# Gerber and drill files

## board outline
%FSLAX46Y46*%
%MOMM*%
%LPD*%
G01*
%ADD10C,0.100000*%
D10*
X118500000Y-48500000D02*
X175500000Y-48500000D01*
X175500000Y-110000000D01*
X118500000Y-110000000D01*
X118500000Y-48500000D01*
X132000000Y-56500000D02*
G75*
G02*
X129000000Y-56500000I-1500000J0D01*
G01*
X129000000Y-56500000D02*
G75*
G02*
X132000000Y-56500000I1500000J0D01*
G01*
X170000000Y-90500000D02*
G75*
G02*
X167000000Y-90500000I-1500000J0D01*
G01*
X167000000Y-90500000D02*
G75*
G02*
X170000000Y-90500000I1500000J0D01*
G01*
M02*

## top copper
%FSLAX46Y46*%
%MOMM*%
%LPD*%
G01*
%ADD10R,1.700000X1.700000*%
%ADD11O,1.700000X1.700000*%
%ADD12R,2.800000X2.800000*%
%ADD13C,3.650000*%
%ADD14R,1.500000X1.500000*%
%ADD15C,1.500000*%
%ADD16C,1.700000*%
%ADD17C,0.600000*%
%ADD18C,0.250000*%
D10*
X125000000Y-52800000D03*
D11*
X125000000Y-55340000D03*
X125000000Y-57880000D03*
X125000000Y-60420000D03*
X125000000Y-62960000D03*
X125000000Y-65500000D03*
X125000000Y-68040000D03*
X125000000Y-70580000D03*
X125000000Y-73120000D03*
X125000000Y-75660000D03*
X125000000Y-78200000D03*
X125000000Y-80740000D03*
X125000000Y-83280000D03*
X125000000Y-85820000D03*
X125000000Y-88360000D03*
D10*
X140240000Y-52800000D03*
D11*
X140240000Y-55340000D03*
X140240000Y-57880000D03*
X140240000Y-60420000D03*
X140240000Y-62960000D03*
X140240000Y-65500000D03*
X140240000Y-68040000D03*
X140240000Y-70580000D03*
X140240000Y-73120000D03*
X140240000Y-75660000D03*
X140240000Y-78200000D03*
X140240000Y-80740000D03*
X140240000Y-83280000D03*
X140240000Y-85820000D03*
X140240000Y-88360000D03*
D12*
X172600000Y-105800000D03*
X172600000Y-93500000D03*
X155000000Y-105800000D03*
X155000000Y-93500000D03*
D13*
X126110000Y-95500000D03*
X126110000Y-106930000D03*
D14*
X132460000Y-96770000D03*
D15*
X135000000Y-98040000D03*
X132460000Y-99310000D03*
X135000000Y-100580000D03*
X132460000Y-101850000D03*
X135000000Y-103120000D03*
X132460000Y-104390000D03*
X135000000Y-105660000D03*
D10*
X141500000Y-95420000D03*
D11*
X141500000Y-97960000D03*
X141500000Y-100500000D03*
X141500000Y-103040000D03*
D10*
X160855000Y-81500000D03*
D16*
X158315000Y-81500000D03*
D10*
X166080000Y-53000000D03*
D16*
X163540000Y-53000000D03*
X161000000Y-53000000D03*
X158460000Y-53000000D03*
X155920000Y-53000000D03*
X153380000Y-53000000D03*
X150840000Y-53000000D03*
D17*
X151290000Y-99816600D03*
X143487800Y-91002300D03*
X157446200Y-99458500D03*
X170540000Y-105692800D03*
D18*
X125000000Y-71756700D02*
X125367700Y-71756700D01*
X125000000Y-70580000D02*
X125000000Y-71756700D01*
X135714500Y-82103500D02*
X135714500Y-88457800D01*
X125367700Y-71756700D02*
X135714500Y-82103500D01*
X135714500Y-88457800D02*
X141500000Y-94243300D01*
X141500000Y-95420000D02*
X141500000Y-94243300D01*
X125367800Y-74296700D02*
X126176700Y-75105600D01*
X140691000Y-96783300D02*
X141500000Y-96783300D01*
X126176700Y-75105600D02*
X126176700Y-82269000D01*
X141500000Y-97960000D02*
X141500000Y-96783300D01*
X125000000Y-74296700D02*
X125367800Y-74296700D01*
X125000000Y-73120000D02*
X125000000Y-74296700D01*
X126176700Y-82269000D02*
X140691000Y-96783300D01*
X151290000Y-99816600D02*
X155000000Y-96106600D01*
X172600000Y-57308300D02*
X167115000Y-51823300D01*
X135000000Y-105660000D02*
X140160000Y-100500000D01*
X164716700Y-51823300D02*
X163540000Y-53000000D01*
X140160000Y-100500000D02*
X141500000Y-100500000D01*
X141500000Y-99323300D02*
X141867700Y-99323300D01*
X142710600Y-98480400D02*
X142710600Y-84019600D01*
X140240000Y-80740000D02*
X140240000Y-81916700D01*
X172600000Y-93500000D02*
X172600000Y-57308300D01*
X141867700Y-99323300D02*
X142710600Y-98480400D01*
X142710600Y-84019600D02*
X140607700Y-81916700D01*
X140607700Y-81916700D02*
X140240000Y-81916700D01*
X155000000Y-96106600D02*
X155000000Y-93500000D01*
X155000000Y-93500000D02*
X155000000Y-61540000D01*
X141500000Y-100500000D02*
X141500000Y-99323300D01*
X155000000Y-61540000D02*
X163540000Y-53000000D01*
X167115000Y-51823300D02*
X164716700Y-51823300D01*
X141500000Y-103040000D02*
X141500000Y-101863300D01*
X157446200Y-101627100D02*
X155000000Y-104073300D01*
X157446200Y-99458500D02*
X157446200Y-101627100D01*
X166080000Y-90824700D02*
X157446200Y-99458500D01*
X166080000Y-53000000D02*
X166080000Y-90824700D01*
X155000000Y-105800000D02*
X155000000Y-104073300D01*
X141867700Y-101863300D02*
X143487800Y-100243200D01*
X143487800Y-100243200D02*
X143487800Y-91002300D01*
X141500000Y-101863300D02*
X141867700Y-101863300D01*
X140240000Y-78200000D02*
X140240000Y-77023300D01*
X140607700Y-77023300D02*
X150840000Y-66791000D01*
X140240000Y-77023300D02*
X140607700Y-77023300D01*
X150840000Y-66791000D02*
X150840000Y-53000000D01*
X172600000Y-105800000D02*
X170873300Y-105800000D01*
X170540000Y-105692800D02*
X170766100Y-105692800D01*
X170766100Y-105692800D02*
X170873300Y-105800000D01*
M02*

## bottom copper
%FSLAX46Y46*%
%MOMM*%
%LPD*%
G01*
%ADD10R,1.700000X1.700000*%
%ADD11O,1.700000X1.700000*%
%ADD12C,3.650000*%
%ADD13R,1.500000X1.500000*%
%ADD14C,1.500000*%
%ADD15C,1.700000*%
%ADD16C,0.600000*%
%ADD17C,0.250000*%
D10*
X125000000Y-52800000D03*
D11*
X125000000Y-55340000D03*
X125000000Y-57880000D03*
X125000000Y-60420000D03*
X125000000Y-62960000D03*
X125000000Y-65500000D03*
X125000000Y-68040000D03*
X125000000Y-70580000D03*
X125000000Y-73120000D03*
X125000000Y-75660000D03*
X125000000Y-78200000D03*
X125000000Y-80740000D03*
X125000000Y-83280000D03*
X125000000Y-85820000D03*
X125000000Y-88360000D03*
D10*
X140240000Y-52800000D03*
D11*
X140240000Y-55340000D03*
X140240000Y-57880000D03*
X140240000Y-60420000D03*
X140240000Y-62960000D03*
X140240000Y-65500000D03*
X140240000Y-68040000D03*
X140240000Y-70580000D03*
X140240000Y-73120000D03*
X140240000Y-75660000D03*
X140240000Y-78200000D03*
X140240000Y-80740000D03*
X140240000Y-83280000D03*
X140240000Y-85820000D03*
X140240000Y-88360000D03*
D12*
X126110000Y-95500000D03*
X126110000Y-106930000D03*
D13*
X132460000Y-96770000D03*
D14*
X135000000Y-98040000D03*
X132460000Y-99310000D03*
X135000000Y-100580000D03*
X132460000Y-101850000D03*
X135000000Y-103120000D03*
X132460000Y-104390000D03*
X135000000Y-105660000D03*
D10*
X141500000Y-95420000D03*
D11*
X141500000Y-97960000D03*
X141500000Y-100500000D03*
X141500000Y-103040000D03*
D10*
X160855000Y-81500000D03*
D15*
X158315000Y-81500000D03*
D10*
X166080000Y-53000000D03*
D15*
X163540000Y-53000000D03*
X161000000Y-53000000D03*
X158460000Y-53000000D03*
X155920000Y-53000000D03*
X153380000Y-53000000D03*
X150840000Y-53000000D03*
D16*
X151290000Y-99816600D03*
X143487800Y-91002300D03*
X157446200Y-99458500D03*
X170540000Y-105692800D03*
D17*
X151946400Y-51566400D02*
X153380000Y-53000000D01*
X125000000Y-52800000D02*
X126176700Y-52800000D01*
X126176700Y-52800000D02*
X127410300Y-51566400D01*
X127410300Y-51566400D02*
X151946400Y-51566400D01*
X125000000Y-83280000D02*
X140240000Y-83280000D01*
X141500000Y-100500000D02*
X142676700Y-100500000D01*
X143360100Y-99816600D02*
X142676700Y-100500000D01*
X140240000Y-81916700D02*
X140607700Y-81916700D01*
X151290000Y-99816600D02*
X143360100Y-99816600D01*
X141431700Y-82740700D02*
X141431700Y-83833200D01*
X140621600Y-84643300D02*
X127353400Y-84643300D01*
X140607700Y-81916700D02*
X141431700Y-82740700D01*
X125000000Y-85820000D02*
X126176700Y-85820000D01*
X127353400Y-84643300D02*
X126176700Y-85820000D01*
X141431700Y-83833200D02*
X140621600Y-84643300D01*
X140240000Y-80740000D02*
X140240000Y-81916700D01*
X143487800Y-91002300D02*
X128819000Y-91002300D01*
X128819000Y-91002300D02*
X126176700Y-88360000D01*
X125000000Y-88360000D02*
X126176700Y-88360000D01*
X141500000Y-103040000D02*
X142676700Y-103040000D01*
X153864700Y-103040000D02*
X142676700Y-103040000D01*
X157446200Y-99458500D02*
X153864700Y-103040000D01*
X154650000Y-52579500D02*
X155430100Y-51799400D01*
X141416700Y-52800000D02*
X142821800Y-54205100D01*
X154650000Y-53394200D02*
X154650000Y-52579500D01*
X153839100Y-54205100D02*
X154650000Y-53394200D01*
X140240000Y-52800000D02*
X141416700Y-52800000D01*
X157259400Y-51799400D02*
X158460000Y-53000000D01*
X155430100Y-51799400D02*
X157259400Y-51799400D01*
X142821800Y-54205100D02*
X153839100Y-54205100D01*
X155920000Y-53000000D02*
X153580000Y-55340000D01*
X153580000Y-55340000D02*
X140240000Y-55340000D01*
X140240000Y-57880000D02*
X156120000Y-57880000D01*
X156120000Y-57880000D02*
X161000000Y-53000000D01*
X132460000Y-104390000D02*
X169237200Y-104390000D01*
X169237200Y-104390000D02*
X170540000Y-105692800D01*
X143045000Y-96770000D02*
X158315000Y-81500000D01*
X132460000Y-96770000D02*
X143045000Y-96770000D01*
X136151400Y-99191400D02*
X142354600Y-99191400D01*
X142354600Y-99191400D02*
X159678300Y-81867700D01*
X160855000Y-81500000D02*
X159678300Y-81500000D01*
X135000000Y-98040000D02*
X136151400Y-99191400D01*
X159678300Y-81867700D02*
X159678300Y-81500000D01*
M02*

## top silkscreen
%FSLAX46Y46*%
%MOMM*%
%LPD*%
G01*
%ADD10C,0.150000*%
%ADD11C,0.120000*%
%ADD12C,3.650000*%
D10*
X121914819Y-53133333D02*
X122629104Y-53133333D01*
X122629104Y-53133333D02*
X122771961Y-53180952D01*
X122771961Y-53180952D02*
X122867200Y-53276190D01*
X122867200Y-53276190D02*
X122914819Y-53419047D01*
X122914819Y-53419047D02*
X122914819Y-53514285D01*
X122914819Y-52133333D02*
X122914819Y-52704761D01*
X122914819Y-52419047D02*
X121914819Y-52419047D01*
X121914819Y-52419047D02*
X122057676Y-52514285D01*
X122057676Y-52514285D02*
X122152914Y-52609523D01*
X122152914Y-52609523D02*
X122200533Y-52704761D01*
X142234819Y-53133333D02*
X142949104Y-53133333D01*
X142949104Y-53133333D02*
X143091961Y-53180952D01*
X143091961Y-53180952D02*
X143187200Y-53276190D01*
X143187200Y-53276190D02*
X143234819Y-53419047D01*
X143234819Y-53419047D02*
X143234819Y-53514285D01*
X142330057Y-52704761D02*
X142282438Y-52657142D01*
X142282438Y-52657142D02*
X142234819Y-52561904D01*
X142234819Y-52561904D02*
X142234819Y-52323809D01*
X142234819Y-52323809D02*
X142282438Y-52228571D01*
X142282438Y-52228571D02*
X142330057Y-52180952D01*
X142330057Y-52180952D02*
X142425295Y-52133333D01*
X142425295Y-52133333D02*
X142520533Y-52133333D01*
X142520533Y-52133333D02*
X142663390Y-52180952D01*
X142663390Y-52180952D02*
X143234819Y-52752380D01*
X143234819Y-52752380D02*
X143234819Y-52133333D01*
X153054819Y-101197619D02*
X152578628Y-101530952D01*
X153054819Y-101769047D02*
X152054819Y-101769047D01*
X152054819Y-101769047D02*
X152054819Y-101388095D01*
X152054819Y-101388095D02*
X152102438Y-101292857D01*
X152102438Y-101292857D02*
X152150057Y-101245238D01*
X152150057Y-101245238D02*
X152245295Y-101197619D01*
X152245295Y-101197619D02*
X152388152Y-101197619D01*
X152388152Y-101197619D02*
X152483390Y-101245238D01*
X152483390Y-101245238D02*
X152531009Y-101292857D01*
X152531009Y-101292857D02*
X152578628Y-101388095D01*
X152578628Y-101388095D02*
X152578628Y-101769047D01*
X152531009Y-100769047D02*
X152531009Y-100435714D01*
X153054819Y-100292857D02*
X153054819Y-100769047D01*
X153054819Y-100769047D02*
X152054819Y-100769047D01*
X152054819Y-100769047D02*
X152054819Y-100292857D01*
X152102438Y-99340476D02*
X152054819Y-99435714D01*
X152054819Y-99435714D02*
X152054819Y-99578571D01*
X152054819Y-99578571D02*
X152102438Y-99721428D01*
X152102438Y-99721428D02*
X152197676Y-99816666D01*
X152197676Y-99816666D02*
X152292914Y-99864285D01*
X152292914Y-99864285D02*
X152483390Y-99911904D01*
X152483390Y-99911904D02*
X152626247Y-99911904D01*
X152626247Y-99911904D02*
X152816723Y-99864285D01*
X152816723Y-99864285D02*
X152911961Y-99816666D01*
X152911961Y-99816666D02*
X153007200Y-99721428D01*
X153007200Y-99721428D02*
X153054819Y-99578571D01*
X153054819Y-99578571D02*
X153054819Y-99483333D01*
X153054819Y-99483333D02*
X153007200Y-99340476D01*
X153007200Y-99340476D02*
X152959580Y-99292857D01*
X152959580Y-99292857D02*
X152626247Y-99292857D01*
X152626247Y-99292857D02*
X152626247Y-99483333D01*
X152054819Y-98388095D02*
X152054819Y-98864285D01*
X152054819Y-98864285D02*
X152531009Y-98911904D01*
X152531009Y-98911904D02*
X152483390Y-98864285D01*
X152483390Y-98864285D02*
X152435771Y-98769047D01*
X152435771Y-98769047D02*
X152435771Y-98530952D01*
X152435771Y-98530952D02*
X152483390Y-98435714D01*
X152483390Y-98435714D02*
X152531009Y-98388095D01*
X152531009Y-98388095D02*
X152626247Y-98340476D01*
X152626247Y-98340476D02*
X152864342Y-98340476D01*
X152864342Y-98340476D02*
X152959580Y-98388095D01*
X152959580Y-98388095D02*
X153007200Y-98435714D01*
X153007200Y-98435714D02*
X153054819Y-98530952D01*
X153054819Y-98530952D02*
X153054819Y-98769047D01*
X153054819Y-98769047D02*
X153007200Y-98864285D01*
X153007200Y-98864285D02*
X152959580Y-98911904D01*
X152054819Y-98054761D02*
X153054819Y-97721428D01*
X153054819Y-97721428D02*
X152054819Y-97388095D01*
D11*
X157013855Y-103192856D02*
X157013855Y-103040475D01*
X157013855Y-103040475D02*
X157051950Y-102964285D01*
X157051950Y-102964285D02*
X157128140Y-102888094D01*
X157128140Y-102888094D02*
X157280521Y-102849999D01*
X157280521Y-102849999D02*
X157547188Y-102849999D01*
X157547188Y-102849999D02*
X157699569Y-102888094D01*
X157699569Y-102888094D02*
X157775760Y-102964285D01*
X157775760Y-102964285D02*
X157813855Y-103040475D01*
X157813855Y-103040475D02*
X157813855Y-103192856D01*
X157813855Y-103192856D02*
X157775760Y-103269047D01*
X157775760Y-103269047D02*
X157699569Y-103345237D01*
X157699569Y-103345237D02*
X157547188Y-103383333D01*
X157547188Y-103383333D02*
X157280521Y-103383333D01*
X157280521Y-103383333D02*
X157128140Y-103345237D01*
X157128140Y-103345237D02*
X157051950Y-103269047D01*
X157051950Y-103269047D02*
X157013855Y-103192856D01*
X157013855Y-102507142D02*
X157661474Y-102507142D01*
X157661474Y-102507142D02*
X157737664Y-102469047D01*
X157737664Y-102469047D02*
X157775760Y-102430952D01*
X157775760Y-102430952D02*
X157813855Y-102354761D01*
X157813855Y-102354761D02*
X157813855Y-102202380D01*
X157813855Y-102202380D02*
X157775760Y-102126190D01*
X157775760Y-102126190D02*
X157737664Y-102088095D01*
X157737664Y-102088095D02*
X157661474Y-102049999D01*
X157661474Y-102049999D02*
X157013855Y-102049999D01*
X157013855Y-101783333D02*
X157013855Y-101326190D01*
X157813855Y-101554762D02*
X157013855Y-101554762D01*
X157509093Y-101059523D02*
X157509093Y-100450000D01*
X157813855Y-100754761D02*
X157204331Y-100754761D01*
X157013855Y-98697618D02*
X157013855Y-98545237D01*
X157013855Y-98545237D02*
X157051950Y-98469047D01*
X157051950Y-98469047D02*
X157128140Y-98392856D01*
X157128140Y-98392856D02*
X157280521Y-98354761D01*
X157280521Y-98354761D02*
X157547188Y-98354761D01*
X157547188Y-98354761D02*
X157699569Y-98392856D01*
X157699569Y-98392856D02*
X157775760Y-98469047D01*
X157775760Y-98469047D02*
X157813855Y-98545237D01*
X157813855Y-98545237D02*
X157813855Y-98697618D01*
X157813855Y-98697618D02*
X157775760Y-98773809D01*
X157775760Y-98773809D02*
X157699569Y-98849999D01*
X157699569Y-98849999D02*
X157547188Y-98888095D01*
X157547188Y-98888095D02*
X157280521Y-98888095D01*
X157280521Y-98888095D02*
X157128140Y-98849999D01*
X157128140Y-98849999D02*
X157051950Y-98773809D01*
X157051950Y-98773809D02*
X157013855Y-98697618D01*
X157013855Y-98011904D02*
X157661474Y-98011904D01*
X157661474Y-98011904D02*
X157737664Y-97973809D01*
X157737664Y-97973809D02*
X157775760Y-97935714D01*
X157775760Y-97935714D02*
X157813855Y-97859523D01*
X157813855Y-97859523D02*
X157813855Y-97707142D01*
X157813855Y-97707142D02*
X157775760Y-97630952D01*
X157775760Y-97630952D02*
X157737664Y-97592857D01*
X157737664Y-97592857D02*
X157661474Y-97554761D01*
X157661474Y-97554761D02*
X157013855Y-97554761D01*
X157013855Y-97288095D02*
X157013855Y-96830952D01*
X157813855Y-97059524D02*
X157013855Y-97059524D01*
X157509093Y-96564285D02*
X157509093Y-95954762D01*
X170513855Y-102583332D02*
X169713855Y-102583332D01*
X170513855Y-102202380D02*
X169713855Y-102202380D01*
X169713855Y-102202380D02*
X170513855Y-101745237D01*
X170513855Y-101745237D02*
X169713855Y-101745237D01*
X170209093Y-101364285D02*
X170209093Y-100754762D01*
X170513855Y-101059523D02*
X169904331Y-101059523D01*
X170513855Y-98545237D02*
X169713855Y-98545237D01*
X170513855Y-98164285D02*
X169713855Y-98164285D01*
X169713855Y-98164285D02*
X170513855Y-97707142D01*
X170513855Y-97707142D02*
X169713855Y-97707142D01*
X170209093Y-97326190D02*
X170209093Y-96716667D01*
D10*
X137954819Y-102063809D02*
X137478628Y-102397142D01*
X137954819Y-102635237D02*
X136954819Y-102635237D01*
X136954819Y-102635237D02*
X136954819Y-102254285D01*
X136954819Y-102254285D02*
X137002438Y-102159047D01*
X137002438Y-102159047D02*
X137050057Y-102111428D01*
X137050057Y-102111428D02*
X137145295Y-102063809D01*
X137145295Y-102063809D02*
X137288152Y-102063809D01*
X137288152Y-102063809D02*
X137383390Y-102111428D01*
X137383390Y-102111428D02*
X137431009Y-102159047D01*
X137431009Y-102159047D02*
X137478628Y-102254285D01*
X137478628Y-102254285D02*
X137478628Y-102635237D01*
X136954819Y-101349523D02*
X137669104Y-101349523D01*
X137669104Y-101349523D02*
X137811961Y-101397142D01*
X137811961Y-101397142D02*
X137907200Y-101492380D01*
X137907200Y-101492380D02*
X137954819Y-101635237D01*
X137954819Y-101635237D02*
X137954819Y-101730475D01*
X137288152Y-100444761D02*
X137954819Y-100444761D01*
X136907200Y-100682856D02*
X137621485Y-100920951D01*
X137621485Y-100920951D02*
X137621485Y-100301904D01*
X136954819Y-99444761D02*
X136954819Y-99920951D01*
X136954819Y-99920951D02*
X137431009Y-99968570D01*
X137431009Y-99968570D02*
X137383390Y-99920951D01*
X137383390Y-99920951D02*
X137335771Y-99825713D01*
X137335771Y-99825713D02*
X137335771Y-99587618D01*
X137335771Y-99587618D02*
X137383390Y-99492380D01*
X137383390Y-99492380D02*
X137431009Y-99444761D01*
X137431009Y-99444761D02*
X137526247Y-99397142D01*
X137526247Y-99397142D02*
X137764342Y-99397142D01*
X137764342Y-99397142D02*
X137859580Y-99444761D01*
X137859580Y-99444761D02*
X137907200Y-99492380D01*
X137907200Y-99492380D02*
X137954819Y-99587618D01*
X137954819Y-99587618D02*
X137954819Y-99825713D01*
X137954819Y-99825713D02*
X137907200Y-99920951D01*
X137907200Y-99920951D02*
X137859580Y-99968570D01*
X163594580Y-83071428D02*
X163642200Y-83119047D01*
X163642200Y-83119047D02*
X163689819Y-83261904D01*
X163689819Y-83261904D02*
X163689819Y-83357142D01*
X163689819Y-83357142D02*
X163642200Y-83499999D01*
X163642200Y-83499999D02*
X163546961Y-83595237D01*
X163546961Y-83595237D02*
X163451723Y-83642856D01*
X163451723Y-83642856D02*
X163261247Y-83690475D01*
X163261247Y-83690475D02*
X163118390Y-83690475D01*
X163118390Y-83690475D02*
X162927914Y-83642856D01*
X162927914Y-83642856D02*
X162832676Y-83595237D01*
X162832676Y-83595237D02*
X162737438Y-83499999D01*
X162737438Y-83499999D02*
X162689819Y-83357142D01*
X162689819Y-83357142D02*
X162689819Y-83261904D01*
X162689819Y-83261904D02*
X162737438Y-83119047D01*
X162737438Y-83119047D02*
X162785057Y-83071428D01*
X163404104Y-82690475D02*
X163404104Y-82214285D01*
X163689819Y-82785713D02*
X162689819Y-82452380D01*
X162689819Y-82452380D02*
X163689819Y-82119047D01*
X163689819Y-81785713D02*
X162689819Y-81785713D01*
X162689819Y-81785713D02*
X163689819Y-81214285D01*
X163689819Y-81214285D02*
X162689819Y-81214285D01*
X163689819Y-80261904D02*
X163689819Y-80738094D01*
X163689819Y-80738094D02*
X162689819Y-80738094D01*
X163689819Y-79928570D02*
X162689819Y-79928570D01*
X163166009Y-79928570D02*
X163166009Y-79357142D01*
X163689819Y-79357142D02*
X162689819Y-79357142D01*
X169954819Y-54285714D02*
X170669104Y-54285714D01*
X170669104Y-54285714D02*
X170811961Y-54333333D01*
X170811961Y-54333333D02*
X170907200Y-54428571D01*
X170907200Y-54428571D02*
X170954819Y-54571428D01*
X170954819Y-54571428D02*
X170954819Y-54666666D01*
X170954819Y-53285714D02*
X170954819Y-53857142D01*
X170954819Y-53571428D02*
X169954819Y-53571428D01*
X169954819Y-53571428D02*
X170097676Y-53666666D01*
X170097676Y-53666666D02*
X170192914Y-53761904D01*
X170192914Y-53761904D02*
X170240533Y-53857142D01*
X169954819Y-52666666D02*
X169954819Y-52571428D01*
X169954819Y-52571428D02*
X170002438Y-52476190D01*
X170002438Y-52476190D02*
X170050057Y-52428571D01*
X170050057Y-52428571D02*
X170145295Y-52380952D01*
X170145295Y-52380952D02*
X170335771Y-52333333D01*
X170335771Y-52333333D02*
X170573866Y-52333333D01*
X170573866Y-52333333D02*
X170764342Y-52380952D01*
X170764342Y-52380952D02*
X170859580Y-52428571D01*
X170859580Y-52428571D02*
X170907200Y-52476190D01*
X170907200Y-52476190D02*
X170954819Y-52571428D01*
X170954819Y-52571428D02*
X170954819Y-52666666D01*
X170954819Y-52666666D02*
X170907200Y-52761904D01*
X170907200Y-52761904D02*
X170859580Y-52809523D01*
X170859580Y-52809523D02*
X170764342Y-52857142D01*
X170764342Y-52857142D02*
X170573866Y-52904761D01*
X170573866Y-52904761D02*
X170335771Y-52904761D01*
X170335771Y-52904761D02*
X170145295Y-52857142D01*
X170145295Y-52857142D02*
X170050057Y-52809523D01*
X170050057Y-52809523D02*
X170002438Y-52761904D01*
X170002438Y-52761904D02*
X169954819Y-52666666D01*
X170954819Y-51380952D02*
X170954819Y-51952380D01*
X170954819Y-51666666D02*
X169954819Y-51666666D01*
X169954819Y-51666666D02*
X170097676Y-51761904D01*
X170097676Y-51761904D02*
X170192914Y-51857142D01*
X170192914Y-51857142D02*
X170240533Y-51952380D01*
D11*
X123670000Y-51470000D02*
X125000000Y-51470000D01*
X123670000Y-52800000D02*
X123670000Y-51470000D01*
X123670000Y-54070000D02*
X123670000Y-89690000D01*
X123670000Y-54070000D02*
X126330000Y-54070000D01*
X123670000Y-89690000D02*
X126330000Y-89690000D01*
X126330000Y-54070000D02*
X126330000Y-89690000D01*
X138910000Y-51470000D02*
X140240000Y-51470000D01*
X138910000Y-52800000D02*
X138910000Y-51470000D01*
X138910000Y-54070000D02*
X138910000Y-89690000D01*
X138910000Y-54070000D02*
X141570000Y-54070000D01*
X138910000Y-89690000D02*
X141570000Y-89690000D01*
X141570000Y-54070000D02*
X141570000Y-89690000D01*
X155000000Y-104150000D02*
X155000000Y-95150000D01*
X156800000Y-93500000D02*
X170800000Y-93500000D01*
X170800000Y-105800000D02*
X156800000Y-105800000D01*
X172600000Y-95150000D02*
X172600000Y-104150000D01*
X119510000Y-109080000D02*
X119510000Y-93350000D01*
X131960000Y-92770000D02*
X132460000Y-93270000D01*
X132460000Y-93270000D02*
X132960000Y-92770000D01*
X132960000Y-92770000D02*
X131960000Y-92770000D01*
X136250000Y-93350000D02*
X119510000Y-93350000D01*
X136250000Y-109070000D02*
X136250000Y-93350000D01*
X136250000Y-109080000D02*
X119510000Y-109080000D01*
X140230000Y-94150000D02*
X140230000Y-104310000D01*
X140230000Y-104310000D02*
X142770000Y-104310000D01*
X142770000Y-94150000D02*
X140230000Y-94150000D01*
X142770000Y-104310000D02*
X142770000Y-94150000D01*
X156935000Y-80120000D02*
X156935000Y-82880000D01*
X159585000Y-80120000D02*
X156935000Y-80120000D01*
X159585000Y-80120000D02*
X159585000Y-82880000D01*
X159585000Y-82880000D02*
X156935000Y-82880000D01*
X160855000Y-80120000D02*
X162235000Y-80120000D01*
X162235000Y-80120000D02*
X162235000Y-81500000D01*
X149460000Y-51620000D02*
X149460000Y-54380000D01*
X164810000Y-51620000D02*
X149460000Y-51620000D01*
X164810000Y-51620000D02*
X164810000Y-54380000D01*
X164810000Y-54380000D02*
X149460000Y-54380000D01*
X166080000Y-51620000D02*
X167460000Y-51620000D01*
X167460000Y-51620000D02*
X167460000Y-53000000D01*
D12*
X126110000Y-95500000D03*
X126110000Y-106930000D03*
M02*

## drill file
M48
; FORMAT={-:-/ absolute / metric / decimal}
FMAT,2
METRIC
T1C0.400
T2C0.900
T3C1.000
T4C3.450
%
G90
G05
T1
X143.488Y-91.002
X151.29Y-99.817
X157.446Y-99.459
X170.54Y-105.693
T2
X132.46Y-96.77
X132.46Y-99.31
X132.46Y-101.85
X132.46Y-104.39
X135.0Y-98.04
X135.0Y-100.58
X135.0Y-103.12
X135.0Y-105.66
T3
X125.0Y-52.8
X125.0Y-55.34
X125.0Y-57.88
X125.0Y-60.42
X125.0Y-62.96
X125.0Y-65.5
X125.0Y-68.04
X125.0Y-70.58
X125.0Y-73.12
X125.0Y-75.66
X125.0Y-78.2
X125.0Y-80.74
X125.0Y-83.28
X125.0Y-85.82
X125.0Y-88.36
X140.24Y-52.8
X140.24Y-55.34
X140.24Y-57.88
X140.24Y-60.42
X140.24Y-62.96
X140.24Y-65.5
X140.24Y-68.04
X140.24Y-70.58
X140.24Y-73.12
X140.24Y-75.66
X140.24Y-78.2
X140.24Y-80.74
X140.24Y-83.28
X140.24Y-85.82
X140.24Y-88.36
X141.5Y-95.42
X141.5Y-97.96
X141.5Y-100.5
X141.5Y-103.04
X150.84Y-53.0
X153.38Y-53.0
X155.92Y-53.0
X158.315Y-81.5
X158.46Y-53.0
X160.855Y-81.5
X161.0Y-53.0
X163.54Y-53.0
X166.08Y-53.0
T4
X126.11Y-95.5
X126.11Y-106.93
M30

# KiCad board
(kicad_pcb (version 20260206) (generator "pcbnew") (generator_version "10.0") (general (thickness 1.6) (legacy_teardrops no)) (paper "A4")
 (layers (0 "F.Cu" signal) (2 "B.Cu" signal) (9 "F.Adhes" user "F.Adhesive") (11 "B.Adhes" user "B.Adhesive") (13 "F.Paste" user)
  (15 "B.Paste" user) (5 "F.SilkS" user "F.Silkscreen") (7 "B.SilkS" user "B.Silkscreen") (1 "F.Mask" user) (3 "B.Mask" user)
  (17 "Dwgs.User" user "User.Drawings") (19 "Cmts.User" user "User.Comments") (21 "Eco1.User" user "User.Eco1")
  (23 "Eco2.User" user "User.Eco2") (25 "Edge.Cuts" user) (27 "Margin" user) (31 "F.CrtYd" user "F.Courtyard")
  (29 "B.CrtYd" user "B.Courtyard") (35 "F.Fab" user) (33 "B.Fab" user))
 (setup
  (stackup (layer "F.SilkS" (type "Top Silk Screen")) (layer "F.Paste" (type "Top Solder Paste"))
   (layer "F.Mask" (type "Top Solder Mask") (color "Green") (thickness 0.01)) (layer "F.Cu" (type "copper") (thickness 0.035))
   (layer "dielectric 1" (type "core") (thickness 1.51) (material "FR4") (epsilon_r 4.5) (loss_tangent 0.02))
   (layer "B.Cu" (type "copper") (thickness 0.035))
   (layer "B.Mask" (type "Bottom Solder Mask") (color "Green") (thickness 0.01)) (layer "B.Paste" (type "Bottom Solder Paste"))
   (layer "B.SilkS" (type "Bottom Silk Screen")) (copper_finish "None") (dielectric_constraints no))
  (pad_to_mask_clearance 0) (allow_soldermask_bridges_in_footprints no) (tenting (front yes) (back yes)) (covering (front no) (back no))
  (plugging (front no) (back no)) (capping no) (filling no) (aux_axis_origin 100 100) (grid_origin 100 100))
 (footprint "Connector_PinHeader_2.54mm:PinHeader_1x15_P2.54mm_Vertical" (layer "F.Cu") (at 125 52.8)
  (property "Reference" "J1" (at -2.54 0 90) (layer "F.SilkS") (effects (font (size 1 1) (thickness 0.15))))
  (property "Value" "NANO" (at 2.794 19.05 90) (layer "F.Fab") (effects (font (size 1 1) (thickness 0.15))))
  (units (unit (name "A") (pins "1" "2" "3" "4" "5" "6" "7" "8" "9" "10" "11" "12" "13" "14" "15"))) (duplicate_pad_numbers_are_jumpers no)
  (fp_line (start -1.33 -1.33) (end 0 -1.33) (stroke (width 0.12) (type solid)) (layer "F.SilkS"))
  (fp_line (start -1.33 0) (end -1.33 -1.33) (stroke (width 0.12) (type solid)) (layer "F.SilkS"))
  (fp_line (start -1.33 1.27) (end -1.33 36.89) (stroke (width 0.12) (type solid)) (layer "F.SilkS"))
  (fp_line (start -1.33 1.27) (end 1.33 1.27) (stroke (width 0.12) (type solid)) (layer "F.SilkS"))
  (fp_line (start -1.33 36.89) (end 1.33 36.89) (stroke (width 0.12) (type solid)) (layer "F.SilkS"))
  (fp_line (start 1.33 1.27) (end 1.33 36.89) (stroke (width 0.12) (type solid)) (layer "F.SilkS"))
  (pad "1" thru_hole rect (at 0 0) (size 1.7 1.7) (drill 1) (layers "*.Cu" "*.Mask") (remove_unused_layers no) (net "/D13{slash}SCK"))
  (pad "2" thru_hole oval (at 0 2.54) (size 1.7 1.7) (drill 1) (layers "*.Cu" "*.Mask") (remove_unused_layers no) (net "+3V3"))
  (pad "3" thru_hole oval (at 0 5.08) (size 1.7 1.7) (drill 1) (layers "*.Cu" "*.Mask") (remove_unused_layers no) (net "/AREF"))
  (pad "4" thru_hole oval (at 0 7.62) (size 1.7 1.7) (drill 1) (layers "*.Cu" "*.Mask") (remove_unused_layers no) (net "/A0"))
  (pad "5" thru_hole oval (at 0 10.16) (size 1.7 1.7) (drill 1) (layers "*.Cu" "*.Mask") (remove_unused_layers no) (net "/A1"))
  (pad "6" thru_hole oval (at 0 12.7) (size 1.7 1.7) (drill 1) (layers "*.Cu" "*.Mask") (remove_unused_layers no) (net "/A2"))
  (pad "7" thru_hole oval (at 0 15.24) (size 1.7 1.7) (drill 1) (layers "*.Cu" "*.Mask") (remove_unused_layers no) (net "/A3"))
  (pad "8" thru_hole oval (at 0 17.78) (size 1.7 1.7) (drill 1) (layers "*.Cu" "*.Mask") (remove_unused_layers no) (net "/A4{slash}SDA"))
  (pad "9" thru_hole oval (at 0 20.32) (size 1.7 1.7) (drill 1) (layers "*.Cu" "*.Mask") (remove_unused_layers no) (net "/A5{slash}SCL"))
  (pad "10" thru_hole oval (at 0 22.86) (size 1.7 1.7) (drill 1) (layers "*.Cu" "*.Mask") (remove_unused_layers no) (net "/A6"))
  (pad "11" thru_hole oval (at 0 25.4) (size 1.7 1.7) (drill 1) (layers "*.Cu" "*.Mask") (remove_unused_layers no) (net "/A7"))
  (pad "12" thru_hole oval (at 0 27.94) (size 1.7 1.7) (drill 1) (layers "*.Cu" "*.Mask") (remove_unused_layers no) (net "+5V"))
  (pad "13" thru_hole oval (at 0 30.48) (size 1.7 1.7) (drill 1) (layers "*.Cu" "*.Mask") (remove_unused_layers no) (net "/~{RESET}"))
  (pad "14" thru_hole oval (at 0 33.02) (size 1.7 1.7) (drill 1) (layers "*.Cu" "*.Mask") (remove_unused_layers no) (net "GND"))
  (pad "15" thru_hole oval (at 0 35.56) (size 1.7 1.7) (drill 1) (layers "*.Cu" "*.Mask") (remove_unused_layers no) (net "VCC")))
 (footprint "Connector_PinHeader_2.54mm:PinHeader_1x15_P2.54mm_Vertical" (layer "F.Cu") (at 140.24 52.8)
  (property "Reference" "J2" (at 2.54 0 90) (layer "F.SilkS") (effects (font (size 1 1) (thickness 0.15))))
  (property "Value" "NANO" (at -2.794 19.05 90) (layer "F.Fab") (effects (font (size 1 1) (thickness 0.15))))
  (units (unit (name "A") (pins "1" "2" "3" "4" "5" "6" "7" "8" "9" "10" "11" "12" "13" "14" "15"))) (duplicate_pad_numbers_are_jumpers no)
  (fp_line (start -1.33 -1.33) (end 0 -1.33) (stroke (width 0.12) (type solid)) (layer "F.SilkS"))
  (fp_line (start -1.33 0) (end -1.33 -1.33) (stroke (width 0.12) (type solid)) (layer "F.SilkS"))
  (fp_line (start -1.33 1.27) (end -1.33 36.89) (stroke (width 0.12) (type solid)) (layer "F.SilkS"))
  (fp_line (start -1.33 1.27) (end 1.33 1.27) (stroke (width 0.12) (type solid)) (layer "F.SilkS"))
  (fp_line (start -1.33 36.89) (end 1.33 36.89) (stroke (width 0.12) (type solid)) (layer "F.SilkS"))
  (fp_line (start 1.33 1.27) (end 1.33 36.89) (stroke (width 0.12) (type solid)) (layer "F.SilkS"))
  (pad "1" thru_hole rect (at 0 0) (size 1.7 1.7) (drill 1) (layers "*.Cu" "*.Mask") (remove_unused_layers no) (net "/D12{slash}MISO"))
  (pad "2" thru_hole oval (at 0 2.54) (size 1.7 1.7) (drill 1) (layers "*.Cu" "*.Mask") (remove_unused_layers no) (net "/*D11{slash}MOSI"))
  (pad "3" thru_hole oval (at 0 5.08) (size 1.7 1.7) (drill 1) (layers "*.Cu" "*.Mask") (remove_unused_layers no) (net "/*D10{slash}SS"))
  (pad "4" thru_hole oval (at 0 7.62) (size 1.7 1.7) (drill 1) (layers "*.Cu" "*.Mask") (remove_unused_layers no) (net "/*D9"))
  (pad "5" thru_hole oval (at 0 10.16) (size 1.7 1.7) (drill 1) (layers "*.Cu" "*.Mask") (remove_unused_layers no) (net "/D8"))
  (pad "6" thru_hole oval (at 0 12.7) (size 1.7 1.7) (drill 1) (layers "*.Cu" "*.Mask") (remove_unused_layers no) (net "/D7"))
  (pad "7" thru_hole oval (at 0 15.24) (size 1.7 1.7) (drill 1) (layers "*.Cu" "*.Mask") (remove_unused_layers no) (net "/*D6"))
  (pad "8" thru_hole oval (at 0 17.78) (size 1.7 1.7) (drill 1) (layers "*.Cu" "*.Mask") (remove_unused_layers no) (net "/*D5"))
  (pad "9" thru_hole oval (at 0 20.32) (size 1.7 1.7) (drill 1) (layers "*.Cu" "*.Mask") (remove_unused_layers no) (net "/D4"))
  (pad "10" thru_hole oval (at 0 22.86) (size 1.7 1.7) (drill 1) (layers "*.Cu" "*.Mask") (remove_unused_layers no) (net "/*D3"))
  (pad "11" thru_hole oval (at 0 25.4) (size 1.7 1.7) (drill 1) (layers "*.Cu" "*.Mask") (remove_unused_layers no) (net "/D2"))
  (pad "12" thru_hole oval (at 0 27.94) (size 1.7 1.7) (drill 1) (layers "*.Cu" "*.Mask") (remove_unused_layers no) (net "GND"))
  (pad "13" thru_hole oval (at 0 30.48) (size 1.7 1.7) (drill 1) (layers "*.Cu" "*.Mask") (remove_unused_layers no) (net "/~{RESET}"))
  (pad "14" thru_hole oval (at 0 33.02) (size 1.7 1.7) (drill 1) (layers "*.Cu" "*.Mask") (remove_unused_layers no) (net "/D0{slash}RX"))
  (pad "15" thru_hole oval (at 0 35.56) (size 1.7 1.7) (drill 1) (layers "*.Cu" "*.Mask") (remove_unused_layers no) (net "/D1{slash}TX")))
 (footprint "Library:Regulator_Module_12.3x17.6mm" (layer "F.Cu") (at 163.8 99.65 90)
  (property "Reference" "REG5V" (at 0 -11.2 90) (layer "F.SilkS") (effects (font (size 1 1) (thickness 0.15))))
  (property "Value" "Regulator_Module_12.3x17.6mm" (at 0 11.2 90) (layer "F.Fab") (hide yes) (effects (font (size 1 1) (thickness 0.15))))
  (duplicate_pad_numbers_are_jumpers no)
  (fp_line (start -4.5 -8.8) (end 4.5 -8.8) (stroke (width 0.12) (type solid)) (layer "F.SilkS"))
  (fp_line (start 6.15 -7) (end 6.15 7) (stroke (width 0.12) (type solid)) (layer "F.SilkS"))
  (fp_line (start -6.15 7) (end -6.15 -7) (stroke (width 0.12) (type solid)) (layer "F.SilkS"))
  (fp_line (start 4.5 8.8) (end -4.5 8.8) (stroke (width 0.12) (type solid)) (layer "F.SilkS"))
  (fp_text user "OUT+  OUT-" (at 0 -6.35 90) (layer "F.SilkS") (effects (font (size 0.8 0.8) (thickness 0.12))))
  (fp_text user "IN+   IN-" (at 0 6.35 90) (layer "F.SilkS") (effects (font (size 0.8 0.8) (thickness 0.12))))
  (pad "1" smd rect (at -6.15 8.8 90) (size 2.8 2.8) (layers "F.Cu" "F.Mask" "F.Paste") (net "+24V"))
  (pad "2" smd rect (at 6.15 8.8 90) (size 2.8 2.8) (layers "F.Cu" "F.Mask" "F.Paste") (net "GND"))
  (pad "3" smd rect (at -6.15 -8.8 90) (size 2.8 2.8) (layers "F.Cu" "F.Mask" "F.Paste") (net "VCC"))
  (pad "4" smd rect (at 6.15 -8.8 90) (size 2.8 2.8) (layers "F.Cu" "F.Mask" "F.Paste") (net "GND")))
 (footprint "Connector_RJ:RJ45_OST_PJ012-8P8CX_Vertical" (layer "F.Cu") (at 132.46 96.77 -90)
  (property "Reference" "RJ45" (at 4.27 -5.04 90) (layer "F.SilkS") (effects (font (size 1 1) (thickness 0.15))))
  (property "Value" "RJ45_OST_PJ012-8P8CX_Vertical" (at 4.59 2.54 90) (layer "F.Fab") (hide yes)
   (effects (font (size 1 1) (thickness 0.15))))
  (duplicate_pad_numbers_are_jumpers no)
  (fp_line (start 12.31 12.95) (end -3.42 12.95) (stroke (width 0.12) (type solid)) (layer "F.SilkS"))
  (fp_line (start -4 0.5) (end -3.5 0) (stroke (width 0.12) (type solid)) (layer "F.SilkS"))
  (fp_line (start -3.5 0) (end -4 -0.5) (stroke (width 0.12) (type solid)) (layer "F.SilkS"))
  (fp_line (start -4 -0.5) (end -4 0.5) (stroke (width 0.12) (type solid)) (layer "F.SilkS"))
  (fp_line (start -3.42 -3.79) (end -3.42 12.95) (stroke (width 0.12) (type solid)) (layer "F.SilkS"))
  (fp_line (start 12.3 -3.79) (end -3.42 -3.79) (stroke (width 0.12) (type solid)) (layer "F.SilkS"))
  (fp_line (start 12.31 -3.79) (end 12.31 12.95) (stroke (width 0.12) (type solid)) (layer "F.SilkS"))
  (pad "" np_thru_hole circle (at -1.27 6.35 270) (size 3.65 3.65) (drill 3.45) (layers "*.Cu" "*.SilkS" "*.Mask"))
  (pad "" np_thru_hole circle (at 10.16 6.35 270) (size 3.65 3.65) (drill 3.45) (layers "*.Cu" "*.SilkS" "*.Mask"))
  (pad "1" thru_hole rect (at 0 0 270) (size 1.5 1.5) (drill 0.9) (layers "*.Cu" "*.Mask") (remove_unused_layers no) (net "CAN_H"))
  (pad "2" thru_hole circle (at 1.27 -2.54 270) (size 1.5 1.5) (drill 0.9) (layers "*.Cu" "*.Mask") (remove_unused_layers no) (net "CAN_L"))
  (pad "3" thru_hole circle (at 2.54 0 270) (size 1.5 1.5) (drill 0.9) (layers "*.Cu" "*.Mask") (remove_unused_layers no))
  (pad "4" thru_hole circle (at 3.81 -2.54 270) (size 1.5 1.5) (drill 0.9) (layers "*.Cu" "*.Mask") (remove_unused_layers no))
  (pad "5" thru_hole circle (at 5.08 0 270) (size 1.5 1.5) (drill 0.9) (layers "*.Cu" "*.Mask") (remove_unused_layers no))
  (pad "6" thru_hole circle (at 6.35 -2.54 270) (size 1.5 1.5) (drill 0.9) (layers "*.Cu" "*.Mask") (remove_unused_layers no))
  (pad "7" thru_hole circle (at 7.62 0 270) (size 1.5 1.5) (drill 0.9) (layers "*.Cu" "*.Mask") (remove_unused_layers no) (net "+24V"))
  (pad "8" thru_hole circle (at 8.89 -2.54 270) (size 1.5 1.5) (drill 0.9) (layers "*.Cu" "*.Mask") (remove_unused_layers no) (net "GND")))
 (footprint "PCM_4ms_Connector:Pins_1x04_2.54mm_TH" (layer "F.Cu") (at 141.5 99.23)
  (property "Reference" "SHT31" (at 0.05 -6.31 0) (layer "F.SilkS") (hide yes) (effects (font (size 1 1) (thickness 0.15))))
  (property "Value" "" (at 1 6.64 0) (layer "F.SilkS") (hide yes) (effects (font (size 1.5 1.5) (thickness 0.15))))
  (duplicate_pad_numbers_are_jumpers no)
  (fp_line (start -1.27 -5.08) (end -1.27 5.08) (stroke (width 0.12) (type solid)) (layer "F.SilkS"))
  (fp_line (start -1.27 5.08) (end 1.27 5.08) (stroke (width 0.12) (type solid)) (layer "F.SilkS"))
  (fp_line (start 1.27 -5.08) (end -1.27 -5.08) (stroke (width 0.12) (type solid)) (layer "F.SilkS"))
  (fp_line (start 1.27 5.08) (end 1.27 -5.08) (stroke (width 0.12) (type solid)) (layer "F.SilkS"))
  (pad "1" thru_hole rect (at 0 -3.81) (size 1.7 1.7) (drill 1) (layers "*.Cu" "*.Mask") (remove_unused_layers no) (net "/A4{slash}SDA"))
  (pad "2" thru_hole oval (at 0 -1.27) (size 1.7 1.7) (drill 1) (layers "*.Cu" "*.Mask") (remove_unused_layers no) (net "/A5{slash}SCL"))
  (pad "3" thru_hole oval (at 0 1.27) (size 1.7 1.7) (drill 1) (layers "*.Cu" "*.Mask") (remove_unused_layers no) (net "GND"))
  (pad "4" thru_hole oval (at 0 3.81) (size 1.7 1.7) (drill 1) (layers "*.Cu" "*.Mask") (remove_unused_layers no) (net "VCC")))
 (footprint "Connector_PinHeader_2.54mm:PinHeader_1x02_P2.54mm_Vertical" (layer "F.Cu") (at 160.855 81.5 -90)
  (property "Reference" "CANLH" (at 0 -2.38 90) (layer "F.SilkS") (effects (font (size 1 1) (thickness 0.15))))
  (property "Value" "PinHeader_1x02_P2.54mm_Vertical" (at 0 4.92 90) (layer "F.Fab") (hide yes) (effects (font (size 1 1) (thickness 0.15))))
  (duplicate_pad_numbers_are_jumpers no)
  (fp_line (start -1.38 3.92) (end 1.38 3.92) (stroke (width 0.12) (type solid)) (layer "F.SilkS"))
  (fp_line (start -1.38 1.27) (end -1.38 3.92) (stroke (width 0.12) (type solid)) (layer "F.SilkS"))
  (fp_line (start -1.38 1.27) (end 1.38 1.27) (stroke (width 0.12) (type solid)) (layer "F.SilkS"))
  (fp_line (start 1.38 1.27) (end 1.38 3.92) (stroke (width 0.12) (type solid)) (layer "F.SilkS"))
  (fp_line (start -1.38 0) (end -1.38 -1.38) (stroke (width 0.12) (type solid)) (layer "F.SilkS"))
  (fp_line (start -1.38 -1.38) (end 0 -1.38) (stroke (width 0.12) (type solid)) (layer "F.SilkS"))
  (pad "1" thru_hole rect (at 0 0 270) (size 1.7 1.7) (drill 1) (layers "*.Cu" "*.Mask") (remove_unused_layers no) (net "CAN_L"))
  (pad "2" thru_hole circle (at 0 2.54 270) (size 1.7 1.7) (drill 1) (layers "*.Cu" "*.Mask") (remove_unused_layers no) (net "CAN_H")))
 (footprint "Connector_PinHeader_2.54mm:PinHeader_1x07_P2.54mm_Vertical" (layer "F.Cu") (at 166.08 53 -90)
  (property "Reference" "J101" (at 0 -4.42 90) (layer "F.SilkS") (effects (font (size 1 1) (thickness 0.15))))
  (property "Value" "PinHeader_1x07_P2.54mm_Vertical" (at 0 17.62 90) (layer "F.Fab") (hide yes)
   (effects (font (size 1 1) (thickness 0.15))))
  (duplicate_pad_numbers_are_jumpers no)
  (fp_line (start -1.38 16.62) (end 1.38 16.62) (stroke (width 0.12) (type solid)) (layer "F.SilkS"))
  (fp_line (start -1.38 1.27) (end -1.38 16.62) (stroke (width 0.12) (type solid)) (layer "F.SilkS"))
  (fp_line (start -1.38 1.27) (end 1.38 1.27) (stroke (width 0.12) (type solid)) (layer "F.SilkS"))
  (fp_line (start 1.38 1.27) (end 1.38 16.62) (stroke (width 0.12) (type solid)) (layer "F.SilkS"))
  (fp_line (start -1.38 0) (end -1.38 -1.38) (stroke (width 0.12) (type solid)) (layer "F.SilkS"))
  (fp_line (start -1.38 -1.38) (end 0 -1.38) (stroke (width 0.12) (type solid)) (layer "F.SilkS"))
  (pad "1" thru_hole rect (at 0 0 270) (size 1.7 1.7) (drill 1) (layers "*.Cu" "*.Mask") (remove_unused_layers no) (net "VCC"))
  (pad "2" thru_hole circle (at 0 2.54 270) (size 1.7 1.7) (drill 1) (layers "*.Cu" "*.Mask") (remove_unused_layers no) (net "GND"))
  (pad "3" thru_hole circle (at 0 5.08 270) (size 1.7 1.7) (drill 1) (layers "*.Cu" "*.Mask") (remove_unused_layers no)
   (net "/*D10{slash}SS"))
  (pad "4" thru_hole circle (at 0 7.62 270) (size 1.7 1.7) (drill 1) (layers "*.Cu" "*.Mask") (remove_unused_layers no)
   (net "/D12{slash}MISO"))
  (pad "5" thru_hole circle (at 0 10.16 270) (size 1.7 1.7) (drill 1) (layers "*.Cu" "*.Mask") (remove_unused_layers no)
   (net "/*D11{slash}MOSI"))
  (pad "6" thru_hole circle (at 0 12.7 270) (size 1.7 1.7) (drill 1) (layers "*.Cu" "*.Mask") (remove_unused_layers no)
   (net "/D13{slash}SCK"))
  (pad "7" thru_hole circle (at 0 15.24 270) (size 1.7 1.7) (drill 1) (layers "*.Cu" "*.Mask") (remove_unused_layers no) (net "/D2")))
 (gr_rect (start 118.5 48.5) (end 175.5 110) (stroke (width 0.1) (type default)) (fill no) (layer "Edge.Cuts"))
 (gr_circle (center 130.5 56.5) (end 130.5 58) (stroke (width 0.1) (type default)) (fill no) (layer "Edge.Cuts"))
 (gr_circle (center 168.5 90.5) (end 167 90.5) (stroke (width 0.1) (type default)) (fill no) (layer "Edge.Cuts"))
 (segment (start 151.9464 51.5664) (end 153.38 53) (width 0.25) (layer "B.Cu") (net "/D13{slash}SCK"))
 (segment (start 125 52.8) (end 126.1767 52.8) (width 0.25) (layer "B.Cu") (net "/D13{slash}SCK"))
 (segment (start 126.1767 52.8) (end 127.4103 51.5664) (width 0.25) (layer "B.Cu") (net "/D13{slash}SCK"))
 (segment (start 127.4103 51.5664) (end 151.9464 51.5664) (width 0.25) (layer "B.Cu") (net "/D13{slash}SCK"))
 (segment (start 125 71.7567) (end 125.3677 71.7567) (width 0.25) (layer "F.Cu") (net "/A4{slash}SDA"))
 (segment (start 125 70.58) (end 125 71.7567) (width 0.25) (layer "F.Cu") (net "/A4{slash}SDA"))
 (segment (start 135.7145 82.1035) (end 135.7145 88.4578) (width 0.25) (layer "F.Cu") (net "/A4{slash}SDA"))
 (segment (start 125.3677 71.7567) (end 135.7145 82.1035) (width 0.25) (layer "F.Cu") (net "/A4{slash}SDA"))
 (segment (start 135.7145 88.4578) (end 141.5 94.2433) (width 0.25) (layer "F.Cu") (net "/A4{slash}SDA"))
 (segment (start 141.5 95.42) (end 141.5 94.2433) (width 0.25) (layer "F.Cu") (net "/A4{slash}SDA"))
 (segment (start 125.3678 74.2967) (end 126.1767 75.1056) (width 0.25) (layer "F.Cu") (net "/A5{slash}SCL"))
 (segment (start 140.691 96.7833) (end 141.5 96.7833) (width 0.25) (layer "F.Cu") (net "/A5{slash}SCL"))
 (segment (start 126.1767 75.1056) (end 126.1767 82.269) (width 0.25) (layer "F.Cu") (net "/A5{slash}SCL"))
 (segment (start 141.5 97.96) (end 141.5 96.7833) (width 0.25) (layer "F.Cu") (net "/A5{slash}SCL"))
 (segment (start 125 74.2967) (end 125.3678 74.2967) (width 0.25) (layer "F.Cu") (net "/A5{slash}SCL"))
 (segment (start 125 73.12) (end 125 74.2967) (width 0.25) (layer "F.Cu") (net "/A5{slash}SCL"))
 (segment (start 126.1767 82.269) (end 140.691 96.7833) (width 0.25) (layer "F.Cu") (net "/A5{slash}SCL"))
 (segment (start 125 83.28) (end 140.24 83.28) (width 0.25) (layer "B.Cu") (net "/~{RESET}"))
 (segment (start 151.29 99.8166) (end 155 96.1066) (width 0.25) (layer "F.Cu") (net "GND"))
 (segment (start 172.6 57.3083) (end 167.115 51.8233) (width 0.25) (layer "F.Cu") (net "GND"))
 (segment (start 135 105.66) (end 140.16 100.5) (width 0.25) (layer "F.Cu") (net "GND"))
 (segment (start 164.7167 51.8233) (end 163.54 53) (width 0.25) (layer "F.Cu") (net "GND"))
 (segment (start 140.16 100.5) (end 141.5 100.5) (width 0.25) (layer "F.Cu") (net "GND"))
 (segment (start 141.5 99.3233) (end 141.8677 99.3233) (width 0.25) (layer "F.Cu") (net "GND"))
 (segment (start 142.7106 98.4804) (end 142.7106 84.0196) (width 0.25) (layer "F.Cu") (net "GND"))
 (segment (start 140.24 80.74) (end 140.24 81.9167) (width 0.25) (layer "F.Cu") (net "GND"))
 (segment (start 172.6 93.5) (end 172.6 57.3083) (width 0.25) (layer "F.Cu") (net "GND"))
 (segment (start 141.8677 99.3233) (end 142.7106 98.4804) (width 0.25) (layer "F.Cu") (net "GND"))
 (segment (start 142.7106 84.0196) (end 140.6077 81.9167) (width 0.25) (layer "F.Cu") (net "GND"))
 (segment (start 140.6077 81.9167) (end 140.24 81.9167) (width 0.25) (layer "F.Cu") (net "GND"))
 (segment (start 155 96.1066) (end 155 93.5) (width 0.25) (layer "F.Cu") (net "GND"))
 (segment (start 155 93.5) (end 155 61.54) (width 0.25) (layer "F.Cu") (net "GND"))
 (segment (start 141.5 100.5) (end 141.5 99.3233) (width 0.25) (layer "F.Cu") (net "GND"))
 (segment (start 155 61.54) (end 163.54 53) (width 0.25) (layer "F.Cu") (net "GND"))
 (segment (start 167.115 51.8233) (end 164.7167 51.8233) (width 0.25) (layer "F.Cu") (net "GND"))
 (via (at 151.29 99.8166) (size 0.6) (drill 0.4) (layers "F.Cu" "B.Cu") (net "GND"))
 (segment (start 141.5 100.5) (end 142.6767 100.5) (width 0.25) (layer "B.Cu") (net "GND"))
 (segment (start 143.3601 99.8166) (end 142.6767 100.5) (width 0.25) (layer "B.Cu") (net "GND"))
 (segment (start 140.24 81.9167) (end 140.6077 81.9167) (width 0.25) (layer "B.Cu") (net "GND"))
 (segment (start 151.29 99.8166) (end 143.3601 99.8166) (width 0.25) (layer "B.Cu") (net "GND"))
 (segment (start 141.4317 82.7407) (end 141.4317 83.8332) (width 0.25) (layer "B.Cu") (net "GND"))
 (segment (start 140.6216 84.6433) (end 127.3534 84.6433) (width 0.25) (layer "B.Cu") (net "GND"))
 (segment (start 140.6077 81.9167) (end 141.4317 82.7407) (width 0.25) (layer "B.Cu") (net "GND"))
 (segment (start 125 85.82) (end 126.1767 85.82) (width 0.25) (layer "B.Cu") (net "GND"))
 (segment (start 127.3534 84.6433) (end 126.1767 85.82) (width 0.25) (layer "B.Cu") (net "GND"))
 (segment (start 141.4317 83.8332) (end 140.6216 84.6433) (width 0.25) (layer "B.Cu") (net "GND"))
 (segment (start 140.24 80.74) (end 140.24 81.9167) (width 0.25) (layer "B.Cu") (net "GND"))
 (segment (start 141.5 103.04) (end 141.5 101.8633) (width 0.25) (layer "F.Cu") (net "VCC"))
 (segment (start 157.4462 101.6271) (end 155 104.0733) (width 0.25) (layer "F.Cu") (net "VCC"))
 (segment (start 157.4462 99.4585) (end 157.4462 101.6271) (width 0.25) (layer "F.Cu") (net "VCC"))
 (segment (start 166.08 90.8247) (end 157.4462 99.4585) (width 0.25) (layer "F.Cu") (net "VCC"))
 (segment (start 166.08 53) (end 166.08 90.8247) (width 0.25) (layer "F.Cu") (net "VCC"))
 (segment (start 155 105.8) (end 155 104.0733) (width 0.25) (layer "F.Cu") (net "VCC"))
 (segment (start 141.8677 101.8633) (end 143.4878 100.2432) (width 0.25) (layer "F.Cu") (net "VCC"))
 (segment (start 143.4878 100.2432) (end 143.4878 91.0023) (width 0.25) (layer "F.Cu") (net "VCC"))
 (segment (start 141.5 101.8633) (end 141.8677 101.8633) (width 0.25) (layer "F.Cu") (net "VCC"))
 (via (at 143.4878 91.0023) (size 0.6) (drill 0.4) (layers "F.Cu" "B.Cu") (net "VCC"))
 (via (at 157.4462 99.4585) (size 0.6) (drill 0.4) (layers "F.Cu" "B.Cu") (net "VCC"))
 (segment (start 143.4878 91.0023) (end 128.819 91.0023) (width 0.25) (layer "B.Cu") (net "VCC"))
 (segment (start 128.819 91.0023) (end 126.1767 88.36) (width 0.25) (layer "B.Cu") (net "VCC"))
 (segment (start 125 88.36) (end 126.1767 88.36) (width 0.25) (layer "B.Cu") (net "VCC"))
 (segment (start 141.5 103.04) (end 142.6767 103.04) (width 0.25) (layer "B.Cu") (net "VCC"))
 (segment (start 153.8647 103.04) (end 142.6767 103.04) (width 0.25) (layer "B.Cu") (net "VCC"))
 (segment (start 157.4462 99.4585) (end 153.8647 103.04) (width 0.25) (layer "B.Cu") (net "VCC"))
 (segment (start 154.65 52.5795) (end 155.4301 51.7994) (width 0.25) (layer "B.Cu") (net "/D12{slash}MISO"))
 (segment (start 141.4167 52.8) (end 142.8218 54.2051) (width 0.25) (layer "B.Cu") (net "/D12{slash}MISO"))
 (segment (start 154.65 53.3942) (end 154.65 52.5795) (width 0.25) (layer "B.Cu") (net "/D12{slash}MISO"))
 (segment (start 153.8391 54.2051) (end 154.65 53.3942) (width 0.25) (layer "B.Cu") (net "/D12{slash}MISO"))
 (segment (start 140.24 52.8) (end 141.4167 52.8) (width 0.25) (layer "B.Cu") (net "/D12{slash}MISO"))
 (segment (start 157.2594 51.7994) (end 158.46 53) (width 0.25) (layer "B.Cu") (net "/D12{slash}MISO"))
 (segment (start 155.4301 51.7994) (end 157.2594 51.7994) (width 0.25) (layer "B.Cu") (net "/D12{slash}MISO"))
 (segment (start 142.8218 54.2051) (end 153.8391 54.2051) (width 0.25) (layer "B.Cu") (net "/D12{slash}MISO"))
 (segment (start 155.92 53) (end 153.58 55.34) (width 0.25) (layer "B.Cu") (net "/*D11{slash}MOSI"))
 (segment (start 153.58 55.34) (end 140.24 55.34) (width 0.25) (layer "B.Cu") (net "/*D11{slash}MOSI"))
 (segment (start 140.24 57.88) (end 156.12 57.88) (width 0.25) (layer "B.Cu") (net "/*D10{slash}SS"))
 (segment (start 156.12 57.88) (end 161 53) (width 0.25) (layer "B.Cu") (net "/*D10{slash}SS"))
 (segment (start 140.24 78.2) (end 140.24 77.0233) (width 0.25) (layer "F.Cu") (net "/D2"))
 (segment (start 140.6077 77.0233) (end 150.84 66.791) (width 0.25) (layer "F.Cu") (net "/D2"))
 (segment (start 140.24 77.0233) (end 140.6077 77.0233) (width 0.25) (layer "F.Cu") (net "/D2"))
 (segment (start 150.84 66.791) (end 150.84 53) (width 0.25) (layer "F.Cu") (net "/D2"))
 (segment (start 172.6 105.8) (end 170.8733 105.8) (width 0.25) (layer "F.Cu") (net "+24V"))
 (segment (start 170.54 105.6928) (end 170.7661 105.6928) (width 0.25) (layer "F.Cu") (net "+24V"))
 (segment (start 170.7661 105.6928) (end 170.8733 105.8) (width 0.25) (layer "F.Cu") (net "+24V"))
 (via (at 170.54 105.6928) (size 0.6) (drill 0.4) (layers "F.Cu" "B.Cu") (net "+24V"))
 (segment (start 132.46 104.39) (end 169.2372 104.39) (width 0.25) (layer "B.Cu") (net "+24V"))
 (segment (start 169.2372 104.39) (end 170.54 105.6928) (width 0.25) (layer "B.Cu") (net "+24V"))
 (segment (start 143.045 96.77) (end 158.315 81.5) (width 0.25) (layer "B.Cu") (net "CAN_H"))
 (segment (start 132.46 96.77) (end 143.045 96.77) (width 0.25) (layer "B.Cu") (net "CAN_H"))
 (segment (start 136.1514 99.1914) (end 142.3546 99.1914) (width 0.25) (layer "B.Cu") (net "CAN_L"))
 (segment (start 142.3546 99.1914) (end 159.6783 81.8677) (width 0.25) (layer "B.Cu") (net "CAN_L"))
 (segment (start 160.855 81.5) (end 159.6783 81.5) (width 0.25) (layer "B.Cu") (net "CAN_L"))
 (segment (start 135 98.04) (end 136.1514 99.1914) (width 0.25) (layer "B.Cu") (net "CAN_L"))
 (segment (start 159.6783 81.8677) (end 159.6783 81.5) (width 0.25) (layer "B.Cu") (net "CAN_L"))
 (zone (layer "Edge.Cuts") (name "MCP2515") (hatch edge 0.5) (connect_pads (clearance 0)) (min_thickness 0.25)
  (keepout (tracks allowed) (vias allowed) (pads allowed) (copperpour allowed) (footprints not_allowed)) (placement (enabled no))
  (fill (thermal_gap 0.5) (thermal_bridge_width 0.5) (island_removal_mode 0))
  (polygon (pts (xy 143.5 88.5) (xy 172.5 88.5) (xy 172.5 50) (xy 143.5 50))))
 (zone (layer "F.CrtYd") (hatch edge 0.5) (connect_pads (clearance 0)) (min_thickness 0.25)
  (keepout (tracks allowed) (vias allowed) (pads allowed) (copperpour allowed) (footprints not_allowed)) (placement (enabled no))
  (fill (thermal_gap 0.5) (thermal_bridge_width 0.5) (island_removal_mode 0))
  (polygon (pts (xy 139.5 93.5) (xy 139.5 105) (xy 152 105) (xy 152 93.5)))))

